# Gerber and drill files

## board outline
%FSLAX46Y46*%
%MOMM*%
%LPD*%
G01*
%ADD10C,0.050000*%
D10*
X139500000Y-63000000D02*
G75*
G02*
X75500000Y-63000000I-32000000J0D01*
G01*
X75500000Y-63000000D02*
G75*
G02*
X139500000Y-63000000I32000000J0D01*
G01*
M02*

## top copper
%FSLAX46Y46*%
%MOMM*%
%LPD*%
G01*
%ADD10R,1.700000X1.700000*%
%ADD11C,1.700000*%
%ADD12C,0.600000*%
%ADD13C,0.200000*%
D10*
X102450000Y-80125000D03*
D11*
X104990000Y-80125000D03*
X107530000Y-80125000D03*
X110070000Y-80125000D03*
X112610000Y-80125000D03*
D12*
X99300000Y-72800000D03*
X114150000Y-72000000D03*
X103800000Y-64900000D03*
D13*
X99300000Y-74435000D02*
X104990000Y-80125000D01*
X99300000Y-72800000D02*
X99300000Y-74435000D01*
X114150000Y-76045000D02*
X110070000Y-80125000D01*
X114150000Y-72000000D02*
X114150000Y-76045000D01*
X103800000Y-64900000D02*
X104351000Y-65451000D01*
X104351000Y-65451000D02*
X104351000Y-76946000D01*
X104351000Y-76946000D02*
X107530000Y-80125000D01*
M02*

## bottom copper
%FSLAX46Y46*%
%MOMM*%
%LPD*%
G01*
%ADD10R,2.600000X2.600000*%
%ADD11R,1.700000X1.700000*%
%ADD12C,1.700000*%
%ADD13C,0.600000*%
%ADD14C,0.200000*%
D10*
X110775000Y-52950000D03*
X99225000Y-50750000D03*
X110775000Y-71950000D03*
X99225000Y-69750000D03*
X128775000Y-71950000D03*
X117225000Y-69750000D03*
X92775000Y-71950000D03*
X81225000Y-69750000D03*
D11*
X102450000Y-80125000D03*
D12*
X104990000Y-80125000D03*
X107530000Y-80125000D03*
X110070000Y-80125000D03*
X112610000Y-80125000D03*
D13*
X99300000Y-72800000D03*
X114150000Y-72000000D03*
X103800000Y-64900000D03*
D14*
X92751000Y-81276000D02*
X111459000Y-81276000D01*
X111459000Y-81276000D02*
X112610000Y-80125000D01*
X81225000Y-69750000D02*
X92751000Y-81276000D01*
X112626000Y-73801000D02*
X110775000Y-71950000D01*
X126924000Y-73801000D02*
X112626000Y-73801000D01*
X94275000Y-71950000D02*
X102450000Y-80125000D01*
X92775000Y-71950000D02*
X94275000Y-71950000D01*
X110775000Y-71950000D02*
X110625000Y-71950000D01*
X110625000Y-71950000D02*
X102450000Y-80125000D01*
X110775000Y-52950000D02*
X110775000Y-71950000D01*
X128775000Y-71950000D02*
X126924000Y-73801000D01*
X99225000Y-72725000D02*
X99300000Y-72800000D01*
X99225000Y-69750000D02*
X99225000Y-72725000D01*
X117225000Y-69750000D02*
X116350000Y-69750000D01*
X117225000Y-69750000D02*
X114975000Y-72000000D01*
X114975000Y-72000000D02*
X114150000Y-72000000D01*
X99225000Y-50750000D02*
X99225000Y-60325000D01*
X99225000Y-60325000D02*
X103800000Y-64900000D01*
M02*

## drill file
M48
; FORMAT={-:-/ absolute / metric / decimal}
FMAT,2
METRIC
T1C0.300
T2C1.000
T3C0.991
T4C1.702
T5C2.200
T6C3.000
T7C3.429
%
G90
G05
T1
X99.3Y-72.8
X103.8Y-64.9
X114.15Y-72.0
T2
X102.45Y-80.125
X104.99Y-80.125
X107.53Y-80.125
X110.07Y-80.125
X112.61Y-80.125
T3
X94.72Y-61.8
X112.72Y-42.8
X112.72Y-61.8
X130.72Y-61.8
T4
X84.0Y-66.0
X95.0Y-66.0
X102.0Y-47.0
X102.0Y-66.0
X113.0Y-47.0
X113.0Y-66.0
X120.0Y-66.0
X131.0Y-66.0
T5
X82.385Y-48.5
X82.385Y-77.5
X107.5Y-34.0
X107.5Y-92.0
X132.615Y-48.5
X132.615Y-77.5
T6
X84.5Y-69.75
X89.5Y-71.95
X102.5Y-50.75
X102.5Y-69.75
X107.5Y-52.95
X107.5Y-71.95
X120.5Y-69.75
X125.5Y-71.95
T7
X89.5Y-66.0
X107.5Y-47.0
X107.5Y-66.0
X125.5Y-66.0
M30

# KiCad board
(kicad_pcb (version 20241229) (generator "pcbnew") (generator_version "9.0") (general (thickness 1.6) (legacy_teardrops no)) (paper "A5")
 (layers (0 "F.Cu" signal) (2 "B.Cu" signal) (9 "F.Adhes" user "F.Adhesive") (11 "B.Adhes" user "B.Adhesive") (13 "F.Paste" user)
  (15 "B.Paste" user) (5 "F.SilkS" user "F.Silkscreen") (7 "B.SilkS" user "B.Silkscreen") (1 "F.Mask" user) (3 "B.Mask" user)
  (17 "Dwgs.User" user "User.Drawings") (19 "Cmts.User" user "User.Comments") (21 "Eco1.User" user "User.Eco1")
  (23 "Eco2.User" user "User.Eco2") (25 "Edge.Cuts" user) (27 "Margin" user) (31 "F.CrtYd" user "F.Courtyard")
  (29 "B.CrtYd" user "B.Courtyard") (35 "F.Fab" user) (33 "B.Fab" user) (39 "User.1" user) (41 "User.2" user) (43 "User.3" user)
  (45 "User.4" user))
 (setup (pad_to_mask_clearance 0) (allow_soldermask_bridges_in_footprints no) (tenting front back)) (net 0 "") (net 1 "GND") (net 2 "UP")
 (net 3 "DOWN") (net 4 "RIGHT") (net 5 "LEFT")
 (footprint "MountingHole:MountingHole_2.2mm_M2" (layer "F.Cu") (at 132.614737 48.5)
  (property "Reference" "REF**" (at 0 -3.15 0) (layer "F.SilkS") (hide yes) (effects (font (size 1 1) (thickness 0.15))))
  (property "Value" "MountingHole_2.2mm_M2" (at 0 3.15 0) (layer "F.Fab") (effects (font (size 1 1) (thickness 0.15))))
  (pad "" np_thru_hole circle (at 0 0) (size 2.2 2.2) (drill 2.2) (layers "*.Cu" "*.Mask")))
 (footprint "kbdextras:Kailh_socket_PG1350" (layer "F.Cu") (at 107.5 47)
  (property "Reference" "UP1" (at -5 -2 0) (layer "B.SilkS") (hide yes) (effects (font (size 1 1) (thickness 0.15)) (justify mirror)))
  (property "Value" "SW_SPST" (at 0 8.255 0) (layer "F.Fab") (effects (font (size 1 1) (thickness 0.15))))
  (pad "" np_thru_hole circle (at -5.5 0) (size 1.7018 1.7018) (drill 1.7018) (layers "*.Cu" "*.Mask"))
  (pad "" np_thru_hole circle (at -5 3.75) (size 3 3) (drill 3) (layers "*.Cu" "*.Mask"))
  (pad "" np_thru_hole circle (at 0 0) (size 3.429 3.429) (drill 3.429) (layers "*.Cu" "*.Mask"))
  (pad "" np_thru_hole circle (at 0 5.95) (size 3 3) (drill 3) (layers "*.Cu" "*.Mask"))
  (pad "" np_thru_hole circle (at 5.22 -4.2) (size 0.9906 0.9906) (drill 0.9906) (layers "*.Cu" "*.Mask"))
  (pad "" np_thru_hole circle (at 5.5 0) (size 1.7018 1.7018) (drill 1.7018) (layers "*.Cu" "*.Mask"))
  (pad "1" smd rect (at 3.275 5.95) (size 2.6 2.6) (layers "B.Cu" "B.Mask" "B.Paste") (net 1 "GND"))
  (pad "2" smd rect (at -8.275 3.75) (size 2.6 2.6) (layers "B.Cu" "B.Mask" "B.Paste") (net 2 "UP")))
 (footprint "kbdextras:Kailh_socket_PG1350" (layer "F.Cu") (at 107.5 66)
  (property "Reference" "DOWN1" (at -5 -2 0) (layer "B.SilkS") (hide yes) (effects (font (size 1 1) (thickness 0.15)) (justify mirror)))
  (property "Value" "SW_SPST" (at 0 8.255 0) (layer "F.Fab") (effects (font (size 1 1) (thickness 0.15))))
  (pad "" np_thru_hole circle (at -5.5 0) (size 1.7018 1.7018) (drill 1.7018) (layers "*.Cu" "*.Mask"))
  (pad "" np_thru_hole circle (at -5 3.75) (size 3 3) (drill 3) (layers "*.Cu" "*.Mask"))
  (pad "" np_thru_hole circle (at 0 0) (size 3.429 3.429) (drill 3.429) (layers "*.Cu" "*.Mask"))
  (pad "" np_thru_hole circle (at 0 5.95) (size 3 3) (drill 3) (layers "*.Cu" "*.Mask"))
  (pad "" np_thru_hole circle (at 5.22 -4.2) (size 0.9906 0.9906) (drill 0.9906) (layers "*.Cu" "*.Mask"))
  (pad "" np_thru_hole circle (at 5.5 0) (size 1.7018 1.7018) (drill 1.7018) (layers "*.Cu" "*.Mask"))
  (pad "1" smd rect (at 3.275 5.95) (size 2.6 2.6) (layers "B.Cu" "B.Mask" "B.Paste") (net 1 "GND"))
  (pad "2" smd rect (at -8.275 3.75) (size 2.6 2.6) (layers "B.Cu" "B.Mask" "B.Paste") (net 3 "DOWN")))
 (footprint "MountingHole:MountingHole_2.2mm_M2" (layer "F.Cu") (at 132.614737 77.5)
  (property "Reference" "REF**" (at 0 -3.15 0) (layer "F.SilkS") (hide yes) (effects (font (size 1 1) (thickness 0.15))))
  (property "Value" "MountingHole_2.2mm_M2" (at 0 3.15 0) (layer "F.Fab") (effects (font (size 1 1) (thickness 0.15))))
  (pad "" np_thru_hole circle (at 0 0) (size 2.2 2.2) (drill 2.2) (layers "*.Cu" "*.Mask")))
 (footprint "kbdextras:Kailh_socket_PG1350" (layer "F.Cu") (at 125.5 66)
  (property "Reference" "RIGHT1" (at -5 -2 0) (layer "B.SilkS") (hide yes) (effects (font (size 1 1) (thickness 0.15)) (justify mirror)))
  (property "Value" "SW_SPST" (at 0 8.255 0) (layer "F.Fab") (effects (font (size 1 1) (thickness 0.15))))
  (pad "" np_thru_hole circle (at -5.5 0) (size 1.7018 1.7018) (drill 1.7018) (layers "*.Cu" "*.Mask"))
  (pad "" np_thru_hole circle (at -5 3.75) (size 3 3) (drill 3) (layers "*.Cu" "*.Mask"))
  (pad "" np_thru_hole circle (at 0 0) (size 3.429 3.429) (drill 3.429) (layers "*.Cu" "*.Mask"))
  (pad "" np_thru_hole circle (at 0 5.95) (size 3 3) (drill 3) (layers "*.Cu" "*.Mask"))
  (pad "" np_thru_hole circle (at 5.22 -4.2) (size 0.9906 0.9906) (drill 0.9906) (layers "*.Cu" "*.Mask"))
  (pad "" np_thru_hole circle (at 5.5 0) (size 1.7018 1.7018) (drill 1.7018) (layers "*.Cu" "*.Mask"))
  (pad "1" smd rect (at 3.275 5.95) (size 2.6 2.6) (layers "B.Cu" "B.Mask" "B.Paste") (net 1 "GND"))
  (pad "2" smd rect (at -8.275 3.75) (size 2.6 2.6) (layers "B.Cu" "B.Mask" "B.Paste") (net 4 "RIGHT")))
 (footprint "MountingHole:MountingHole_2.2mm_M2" (layer "F.Cu") (at 82.385263 77.5)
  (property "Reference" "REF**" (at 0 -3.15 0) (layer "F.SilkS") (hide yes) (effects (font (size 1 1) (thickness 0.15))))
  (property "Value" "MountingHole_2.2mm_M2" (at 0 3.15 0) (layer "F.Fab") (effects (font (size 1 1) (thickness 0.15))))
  (pad "" np_thru_hole circle (at 0 0) (size 2.2 2.2) (drill 2.2) (layers "*.Cu" "*.Mask")))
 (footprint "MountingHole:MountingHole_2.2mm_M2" (layer "F.Cu") (at 107.5 34)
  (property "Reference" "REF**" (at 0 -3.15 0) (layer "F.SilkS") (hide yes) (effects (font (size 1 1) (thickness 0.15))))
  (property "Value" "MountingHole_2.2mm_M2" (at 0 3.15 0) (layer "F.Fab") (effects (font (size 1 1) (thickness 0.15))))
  (pad "" np_thru_hole circle (at 0 0) (size 2.2 2.2) (drill 2.2) (layers "*.Cu" "*.Mask")))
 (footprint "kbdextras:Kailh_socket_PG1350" (layer "F.Cu") (at 89.5 66)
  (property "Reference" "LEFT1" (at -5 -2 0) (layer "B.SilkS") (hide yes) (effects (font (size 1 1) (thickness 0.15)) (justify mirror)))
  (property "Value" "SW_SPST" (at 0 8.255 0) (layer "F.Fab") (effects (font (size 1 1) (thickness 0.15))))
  (pad "" np_thru_hole circle (at -5.5 0) (size 1.7018 1.7018) (drill 1.7018) (layers "*.Cu" "*.Mask"))
  (pad "" np_thru_hole circle (at -5 3.75) (size 3 3) (drill 3) (layers "*.Cu" "*.Mask"))
  (pad "" np_thru_hole circle (at 0 0) (size 3.429 3.429) (drill 3.429) (layers "*.Cu" "*.Mask"))
  (pad "" np_thru_hole circle (at 0 5.95) (size 3 3) (drill 3) (layers "*.Cu" "*.Mask"))
  (pad "" np_thru_hole circle (at 5.22 -4.2) (size 0.9906 0.9906) (drill 0.9906) (layers "*.Cu" "*.Mask"))
  (pad "" np_thru_hole circle (at 5.5 0) (size 1.7018 1.7018) (drill 1.7018) (layers "*.Cu" "*.Mask"))
  (pad "1" smd rect (at 3.275 5.95) (size 2.6 2.6) (layers "B.Cu" "B.Mask" "B.Paste") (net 1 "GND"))
  (pad "2" smd rect (at -8.275 3.75) (size 2.6 2.6) (layers "B.Cu" "B.Mask" "B.Paste") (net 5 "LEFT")))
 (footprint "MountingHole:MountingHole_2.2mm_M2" (layer "F.Cu") (at 107.5 92)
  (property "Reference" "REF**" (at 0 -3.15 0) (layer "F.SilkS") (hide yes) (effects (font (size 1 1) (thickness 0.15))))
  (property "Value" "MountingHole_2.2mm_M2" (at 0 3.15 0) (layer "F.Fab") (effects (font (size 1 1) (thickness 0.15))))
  (pad "" np_thru_hole circle (at 0 0) (size 2.2 2.2) (drill 2.2) (layers "*.Cu" "*.Mask")))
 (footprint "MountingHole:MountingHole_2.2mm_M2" (layer "F.Cu") (at 82.385263 48.5)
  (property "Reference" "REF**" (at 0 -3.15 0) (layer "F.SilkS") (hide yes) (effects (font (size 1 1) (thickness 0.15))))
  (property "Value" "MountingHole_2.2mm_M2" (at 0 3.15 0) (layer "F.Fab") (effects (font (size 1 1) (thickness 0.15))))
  (pad "" np_thru_hole circle (at 0 0) (size 2.2 2.2) (drill 2.2) (layers "*.Cu" "*.Mask")))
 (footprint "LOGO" (layer "B.Cu") (at 101.31 51.71)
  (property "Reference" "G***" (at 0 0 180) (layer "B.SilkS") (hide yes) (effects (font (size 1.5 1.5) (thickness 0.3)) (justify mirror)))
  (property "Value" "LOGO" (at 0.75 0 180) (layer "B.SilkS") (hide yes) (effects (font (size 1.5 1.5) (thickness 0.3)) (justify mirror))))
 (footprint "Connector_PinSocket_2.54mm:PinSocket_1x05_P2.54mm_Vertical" (layer "B.Cu") (at 102.45 80.125 -90)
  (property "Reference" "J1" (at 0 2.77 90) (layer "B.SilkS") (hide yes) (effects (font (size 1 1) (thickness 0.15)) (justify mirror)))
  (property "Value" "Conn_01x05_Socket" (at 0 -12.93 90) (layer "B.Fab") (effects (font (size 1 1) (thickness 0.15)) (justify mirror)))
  (pad "1" thru_hole rect (at 0 0 270) (size 1.7 1.7) (drill 1) (layers "*.Cu" "*.Mask") (remove_unused_layers no) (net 1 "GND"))
  (pad "2" thru_hole circle (at 0 -2.54 270) (size 1.7 1.7) (drill 1) (layers "*.Cu" "*.Mask") (remove_unused_layers no) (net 3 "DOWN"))
  (pad "3" thru_hole circle (at 0 -5.08 270) (size 1.7 1.7) (drill 1) (layers "*.Cu" "*.Mask") (remove_unused_layers no) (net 2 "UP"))
  (pad "4" thru_hole circle (at 0 -7.62 270) (size 1.7 1.7) (drill 1) (layers "*.Cu" "*.Mask") (remove_unused_layers no) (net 4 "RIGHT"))
  (pad "5" thru_hole circle (at 0 -10.16 270) (size 1.7 1.7) (drill 1) (layers "*.Cu" "*.Mask") (remove_unused_layers no) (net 5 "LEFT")))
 (gr_circle (center 107.5 63) (end 139.5 63) (stroke (width 0.05) (type solid)) (fill no) (layer "Edge.Cuts"))
 (segment (start 92.751 81.276) (end 111.459 81.276) (width 0.2) (layer "B.Cu") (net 5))
 (segment (start 111.459 81.276) (end 112.61 80.125) (width 0.2) (layer "B.Cu") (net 5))
 (segment (start 81.225 69.75) (end 92.751 81.276) (width 0.2) (layer "B.Cu") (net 5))
 (segment (start 112.626 73.801) (end 110.775 71.95) (width 0.2) (layer "B.Cu") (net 1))
 (segment (start 126.924 73.801) (end 112.626 73.801) (width 0.2) (layer "B.Cu") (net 1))
 (segment (start 94.275 71.95) (end 102.45 80.125) (width 0.2) (layer "B.Cu") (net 1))
 (segment (start 92.775 71.95) (end 94.275 71.95) (width 0.2) (layer "B.Cu") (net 1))
 (segment (start 110.775 71.95) (end 110.625 71.95) (width 0.2) (layer "B.Cu") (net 1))
 (segment (start 110.625 71.95) (end 102.45 80.125) (width 0.2) (layer "B.Cu") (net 1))
 (segment (start 110.775 52.95) (end 110.775 71.95) (width 0.2) (layer "B.Cu") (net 1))
 (segment (start 128.775 71.95) (end 126.924 73.801) (width 0.2) (layer "B.Cu") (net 1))
 (segment (start 99.3 74.435) (end 104.99 80.125) (width 0.2) (layer "F.Cu") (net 3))
 (segment (start 99.3 72.8) (end 99.3 74.435) (width 0.2) (layer "F.Cu") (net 3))
 (via (at 99.3 72.8) (size 0.6) (drill 0.3) (layers "F.Cu" "B.Cu") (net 3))
 (segment (start 99.225 72.725) (end 99.3 72.8) (width 0.2) (layer "B.Cu") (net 3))
 (segment (start 99.225 69.75) (end 99.225 72.725) (width 0.2) (layer "B.Cu") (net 3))
 (segment (start 114.15 76.045) (end 110.07 80.125) (width 0.2) (layer "F.Cu") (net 4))
 (segment (start 114.15 72) (end 114.15 76.045) (width 0.2) (layer "F.Cu") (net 4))
 (via (at 114.15 72) (size 0.6) (drill 0.3) (layers "F.Cu" "B.Cu") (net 4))
 (segment (start 117.225 69.75) (end 116.35 69.75) (width 0.2) (layer "B.Cu") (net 4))
 (segment (start 117.225 69.75) (end 114.975 72) (width 0.2) (layer "B.Cu") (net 4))
 (segment (start 114.975 72) (end 114.15 72) (width 0.2) (layer "B.Cu") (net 4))
 (segment (start 103.8 64.9) (end 104.351 65.451) (width 0.2) (layer "F.Cu") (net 2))
 (segment (start 104.351 65.451) (end 104.351 76.946) (width 0.2) (layer "F.Cu") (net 2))
 (segment (start 104.351 76.946) (end 107.53 80.125) (width 0.2) (layer "F.Cu") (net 2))
 (via (at 103.8 64.9) (size 0.6) (drill 0.3) (layers "F.Cu" "B.Cu") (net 2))
 (segment (start 99.225 50.75) (end 99.225 60.325) (width 0.2) (layer "B.Cu") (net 2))
 (segment (start 99.225 60.325) (end 103.8 64.9) (width 0.2) (layer "B.Cu") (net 2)))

